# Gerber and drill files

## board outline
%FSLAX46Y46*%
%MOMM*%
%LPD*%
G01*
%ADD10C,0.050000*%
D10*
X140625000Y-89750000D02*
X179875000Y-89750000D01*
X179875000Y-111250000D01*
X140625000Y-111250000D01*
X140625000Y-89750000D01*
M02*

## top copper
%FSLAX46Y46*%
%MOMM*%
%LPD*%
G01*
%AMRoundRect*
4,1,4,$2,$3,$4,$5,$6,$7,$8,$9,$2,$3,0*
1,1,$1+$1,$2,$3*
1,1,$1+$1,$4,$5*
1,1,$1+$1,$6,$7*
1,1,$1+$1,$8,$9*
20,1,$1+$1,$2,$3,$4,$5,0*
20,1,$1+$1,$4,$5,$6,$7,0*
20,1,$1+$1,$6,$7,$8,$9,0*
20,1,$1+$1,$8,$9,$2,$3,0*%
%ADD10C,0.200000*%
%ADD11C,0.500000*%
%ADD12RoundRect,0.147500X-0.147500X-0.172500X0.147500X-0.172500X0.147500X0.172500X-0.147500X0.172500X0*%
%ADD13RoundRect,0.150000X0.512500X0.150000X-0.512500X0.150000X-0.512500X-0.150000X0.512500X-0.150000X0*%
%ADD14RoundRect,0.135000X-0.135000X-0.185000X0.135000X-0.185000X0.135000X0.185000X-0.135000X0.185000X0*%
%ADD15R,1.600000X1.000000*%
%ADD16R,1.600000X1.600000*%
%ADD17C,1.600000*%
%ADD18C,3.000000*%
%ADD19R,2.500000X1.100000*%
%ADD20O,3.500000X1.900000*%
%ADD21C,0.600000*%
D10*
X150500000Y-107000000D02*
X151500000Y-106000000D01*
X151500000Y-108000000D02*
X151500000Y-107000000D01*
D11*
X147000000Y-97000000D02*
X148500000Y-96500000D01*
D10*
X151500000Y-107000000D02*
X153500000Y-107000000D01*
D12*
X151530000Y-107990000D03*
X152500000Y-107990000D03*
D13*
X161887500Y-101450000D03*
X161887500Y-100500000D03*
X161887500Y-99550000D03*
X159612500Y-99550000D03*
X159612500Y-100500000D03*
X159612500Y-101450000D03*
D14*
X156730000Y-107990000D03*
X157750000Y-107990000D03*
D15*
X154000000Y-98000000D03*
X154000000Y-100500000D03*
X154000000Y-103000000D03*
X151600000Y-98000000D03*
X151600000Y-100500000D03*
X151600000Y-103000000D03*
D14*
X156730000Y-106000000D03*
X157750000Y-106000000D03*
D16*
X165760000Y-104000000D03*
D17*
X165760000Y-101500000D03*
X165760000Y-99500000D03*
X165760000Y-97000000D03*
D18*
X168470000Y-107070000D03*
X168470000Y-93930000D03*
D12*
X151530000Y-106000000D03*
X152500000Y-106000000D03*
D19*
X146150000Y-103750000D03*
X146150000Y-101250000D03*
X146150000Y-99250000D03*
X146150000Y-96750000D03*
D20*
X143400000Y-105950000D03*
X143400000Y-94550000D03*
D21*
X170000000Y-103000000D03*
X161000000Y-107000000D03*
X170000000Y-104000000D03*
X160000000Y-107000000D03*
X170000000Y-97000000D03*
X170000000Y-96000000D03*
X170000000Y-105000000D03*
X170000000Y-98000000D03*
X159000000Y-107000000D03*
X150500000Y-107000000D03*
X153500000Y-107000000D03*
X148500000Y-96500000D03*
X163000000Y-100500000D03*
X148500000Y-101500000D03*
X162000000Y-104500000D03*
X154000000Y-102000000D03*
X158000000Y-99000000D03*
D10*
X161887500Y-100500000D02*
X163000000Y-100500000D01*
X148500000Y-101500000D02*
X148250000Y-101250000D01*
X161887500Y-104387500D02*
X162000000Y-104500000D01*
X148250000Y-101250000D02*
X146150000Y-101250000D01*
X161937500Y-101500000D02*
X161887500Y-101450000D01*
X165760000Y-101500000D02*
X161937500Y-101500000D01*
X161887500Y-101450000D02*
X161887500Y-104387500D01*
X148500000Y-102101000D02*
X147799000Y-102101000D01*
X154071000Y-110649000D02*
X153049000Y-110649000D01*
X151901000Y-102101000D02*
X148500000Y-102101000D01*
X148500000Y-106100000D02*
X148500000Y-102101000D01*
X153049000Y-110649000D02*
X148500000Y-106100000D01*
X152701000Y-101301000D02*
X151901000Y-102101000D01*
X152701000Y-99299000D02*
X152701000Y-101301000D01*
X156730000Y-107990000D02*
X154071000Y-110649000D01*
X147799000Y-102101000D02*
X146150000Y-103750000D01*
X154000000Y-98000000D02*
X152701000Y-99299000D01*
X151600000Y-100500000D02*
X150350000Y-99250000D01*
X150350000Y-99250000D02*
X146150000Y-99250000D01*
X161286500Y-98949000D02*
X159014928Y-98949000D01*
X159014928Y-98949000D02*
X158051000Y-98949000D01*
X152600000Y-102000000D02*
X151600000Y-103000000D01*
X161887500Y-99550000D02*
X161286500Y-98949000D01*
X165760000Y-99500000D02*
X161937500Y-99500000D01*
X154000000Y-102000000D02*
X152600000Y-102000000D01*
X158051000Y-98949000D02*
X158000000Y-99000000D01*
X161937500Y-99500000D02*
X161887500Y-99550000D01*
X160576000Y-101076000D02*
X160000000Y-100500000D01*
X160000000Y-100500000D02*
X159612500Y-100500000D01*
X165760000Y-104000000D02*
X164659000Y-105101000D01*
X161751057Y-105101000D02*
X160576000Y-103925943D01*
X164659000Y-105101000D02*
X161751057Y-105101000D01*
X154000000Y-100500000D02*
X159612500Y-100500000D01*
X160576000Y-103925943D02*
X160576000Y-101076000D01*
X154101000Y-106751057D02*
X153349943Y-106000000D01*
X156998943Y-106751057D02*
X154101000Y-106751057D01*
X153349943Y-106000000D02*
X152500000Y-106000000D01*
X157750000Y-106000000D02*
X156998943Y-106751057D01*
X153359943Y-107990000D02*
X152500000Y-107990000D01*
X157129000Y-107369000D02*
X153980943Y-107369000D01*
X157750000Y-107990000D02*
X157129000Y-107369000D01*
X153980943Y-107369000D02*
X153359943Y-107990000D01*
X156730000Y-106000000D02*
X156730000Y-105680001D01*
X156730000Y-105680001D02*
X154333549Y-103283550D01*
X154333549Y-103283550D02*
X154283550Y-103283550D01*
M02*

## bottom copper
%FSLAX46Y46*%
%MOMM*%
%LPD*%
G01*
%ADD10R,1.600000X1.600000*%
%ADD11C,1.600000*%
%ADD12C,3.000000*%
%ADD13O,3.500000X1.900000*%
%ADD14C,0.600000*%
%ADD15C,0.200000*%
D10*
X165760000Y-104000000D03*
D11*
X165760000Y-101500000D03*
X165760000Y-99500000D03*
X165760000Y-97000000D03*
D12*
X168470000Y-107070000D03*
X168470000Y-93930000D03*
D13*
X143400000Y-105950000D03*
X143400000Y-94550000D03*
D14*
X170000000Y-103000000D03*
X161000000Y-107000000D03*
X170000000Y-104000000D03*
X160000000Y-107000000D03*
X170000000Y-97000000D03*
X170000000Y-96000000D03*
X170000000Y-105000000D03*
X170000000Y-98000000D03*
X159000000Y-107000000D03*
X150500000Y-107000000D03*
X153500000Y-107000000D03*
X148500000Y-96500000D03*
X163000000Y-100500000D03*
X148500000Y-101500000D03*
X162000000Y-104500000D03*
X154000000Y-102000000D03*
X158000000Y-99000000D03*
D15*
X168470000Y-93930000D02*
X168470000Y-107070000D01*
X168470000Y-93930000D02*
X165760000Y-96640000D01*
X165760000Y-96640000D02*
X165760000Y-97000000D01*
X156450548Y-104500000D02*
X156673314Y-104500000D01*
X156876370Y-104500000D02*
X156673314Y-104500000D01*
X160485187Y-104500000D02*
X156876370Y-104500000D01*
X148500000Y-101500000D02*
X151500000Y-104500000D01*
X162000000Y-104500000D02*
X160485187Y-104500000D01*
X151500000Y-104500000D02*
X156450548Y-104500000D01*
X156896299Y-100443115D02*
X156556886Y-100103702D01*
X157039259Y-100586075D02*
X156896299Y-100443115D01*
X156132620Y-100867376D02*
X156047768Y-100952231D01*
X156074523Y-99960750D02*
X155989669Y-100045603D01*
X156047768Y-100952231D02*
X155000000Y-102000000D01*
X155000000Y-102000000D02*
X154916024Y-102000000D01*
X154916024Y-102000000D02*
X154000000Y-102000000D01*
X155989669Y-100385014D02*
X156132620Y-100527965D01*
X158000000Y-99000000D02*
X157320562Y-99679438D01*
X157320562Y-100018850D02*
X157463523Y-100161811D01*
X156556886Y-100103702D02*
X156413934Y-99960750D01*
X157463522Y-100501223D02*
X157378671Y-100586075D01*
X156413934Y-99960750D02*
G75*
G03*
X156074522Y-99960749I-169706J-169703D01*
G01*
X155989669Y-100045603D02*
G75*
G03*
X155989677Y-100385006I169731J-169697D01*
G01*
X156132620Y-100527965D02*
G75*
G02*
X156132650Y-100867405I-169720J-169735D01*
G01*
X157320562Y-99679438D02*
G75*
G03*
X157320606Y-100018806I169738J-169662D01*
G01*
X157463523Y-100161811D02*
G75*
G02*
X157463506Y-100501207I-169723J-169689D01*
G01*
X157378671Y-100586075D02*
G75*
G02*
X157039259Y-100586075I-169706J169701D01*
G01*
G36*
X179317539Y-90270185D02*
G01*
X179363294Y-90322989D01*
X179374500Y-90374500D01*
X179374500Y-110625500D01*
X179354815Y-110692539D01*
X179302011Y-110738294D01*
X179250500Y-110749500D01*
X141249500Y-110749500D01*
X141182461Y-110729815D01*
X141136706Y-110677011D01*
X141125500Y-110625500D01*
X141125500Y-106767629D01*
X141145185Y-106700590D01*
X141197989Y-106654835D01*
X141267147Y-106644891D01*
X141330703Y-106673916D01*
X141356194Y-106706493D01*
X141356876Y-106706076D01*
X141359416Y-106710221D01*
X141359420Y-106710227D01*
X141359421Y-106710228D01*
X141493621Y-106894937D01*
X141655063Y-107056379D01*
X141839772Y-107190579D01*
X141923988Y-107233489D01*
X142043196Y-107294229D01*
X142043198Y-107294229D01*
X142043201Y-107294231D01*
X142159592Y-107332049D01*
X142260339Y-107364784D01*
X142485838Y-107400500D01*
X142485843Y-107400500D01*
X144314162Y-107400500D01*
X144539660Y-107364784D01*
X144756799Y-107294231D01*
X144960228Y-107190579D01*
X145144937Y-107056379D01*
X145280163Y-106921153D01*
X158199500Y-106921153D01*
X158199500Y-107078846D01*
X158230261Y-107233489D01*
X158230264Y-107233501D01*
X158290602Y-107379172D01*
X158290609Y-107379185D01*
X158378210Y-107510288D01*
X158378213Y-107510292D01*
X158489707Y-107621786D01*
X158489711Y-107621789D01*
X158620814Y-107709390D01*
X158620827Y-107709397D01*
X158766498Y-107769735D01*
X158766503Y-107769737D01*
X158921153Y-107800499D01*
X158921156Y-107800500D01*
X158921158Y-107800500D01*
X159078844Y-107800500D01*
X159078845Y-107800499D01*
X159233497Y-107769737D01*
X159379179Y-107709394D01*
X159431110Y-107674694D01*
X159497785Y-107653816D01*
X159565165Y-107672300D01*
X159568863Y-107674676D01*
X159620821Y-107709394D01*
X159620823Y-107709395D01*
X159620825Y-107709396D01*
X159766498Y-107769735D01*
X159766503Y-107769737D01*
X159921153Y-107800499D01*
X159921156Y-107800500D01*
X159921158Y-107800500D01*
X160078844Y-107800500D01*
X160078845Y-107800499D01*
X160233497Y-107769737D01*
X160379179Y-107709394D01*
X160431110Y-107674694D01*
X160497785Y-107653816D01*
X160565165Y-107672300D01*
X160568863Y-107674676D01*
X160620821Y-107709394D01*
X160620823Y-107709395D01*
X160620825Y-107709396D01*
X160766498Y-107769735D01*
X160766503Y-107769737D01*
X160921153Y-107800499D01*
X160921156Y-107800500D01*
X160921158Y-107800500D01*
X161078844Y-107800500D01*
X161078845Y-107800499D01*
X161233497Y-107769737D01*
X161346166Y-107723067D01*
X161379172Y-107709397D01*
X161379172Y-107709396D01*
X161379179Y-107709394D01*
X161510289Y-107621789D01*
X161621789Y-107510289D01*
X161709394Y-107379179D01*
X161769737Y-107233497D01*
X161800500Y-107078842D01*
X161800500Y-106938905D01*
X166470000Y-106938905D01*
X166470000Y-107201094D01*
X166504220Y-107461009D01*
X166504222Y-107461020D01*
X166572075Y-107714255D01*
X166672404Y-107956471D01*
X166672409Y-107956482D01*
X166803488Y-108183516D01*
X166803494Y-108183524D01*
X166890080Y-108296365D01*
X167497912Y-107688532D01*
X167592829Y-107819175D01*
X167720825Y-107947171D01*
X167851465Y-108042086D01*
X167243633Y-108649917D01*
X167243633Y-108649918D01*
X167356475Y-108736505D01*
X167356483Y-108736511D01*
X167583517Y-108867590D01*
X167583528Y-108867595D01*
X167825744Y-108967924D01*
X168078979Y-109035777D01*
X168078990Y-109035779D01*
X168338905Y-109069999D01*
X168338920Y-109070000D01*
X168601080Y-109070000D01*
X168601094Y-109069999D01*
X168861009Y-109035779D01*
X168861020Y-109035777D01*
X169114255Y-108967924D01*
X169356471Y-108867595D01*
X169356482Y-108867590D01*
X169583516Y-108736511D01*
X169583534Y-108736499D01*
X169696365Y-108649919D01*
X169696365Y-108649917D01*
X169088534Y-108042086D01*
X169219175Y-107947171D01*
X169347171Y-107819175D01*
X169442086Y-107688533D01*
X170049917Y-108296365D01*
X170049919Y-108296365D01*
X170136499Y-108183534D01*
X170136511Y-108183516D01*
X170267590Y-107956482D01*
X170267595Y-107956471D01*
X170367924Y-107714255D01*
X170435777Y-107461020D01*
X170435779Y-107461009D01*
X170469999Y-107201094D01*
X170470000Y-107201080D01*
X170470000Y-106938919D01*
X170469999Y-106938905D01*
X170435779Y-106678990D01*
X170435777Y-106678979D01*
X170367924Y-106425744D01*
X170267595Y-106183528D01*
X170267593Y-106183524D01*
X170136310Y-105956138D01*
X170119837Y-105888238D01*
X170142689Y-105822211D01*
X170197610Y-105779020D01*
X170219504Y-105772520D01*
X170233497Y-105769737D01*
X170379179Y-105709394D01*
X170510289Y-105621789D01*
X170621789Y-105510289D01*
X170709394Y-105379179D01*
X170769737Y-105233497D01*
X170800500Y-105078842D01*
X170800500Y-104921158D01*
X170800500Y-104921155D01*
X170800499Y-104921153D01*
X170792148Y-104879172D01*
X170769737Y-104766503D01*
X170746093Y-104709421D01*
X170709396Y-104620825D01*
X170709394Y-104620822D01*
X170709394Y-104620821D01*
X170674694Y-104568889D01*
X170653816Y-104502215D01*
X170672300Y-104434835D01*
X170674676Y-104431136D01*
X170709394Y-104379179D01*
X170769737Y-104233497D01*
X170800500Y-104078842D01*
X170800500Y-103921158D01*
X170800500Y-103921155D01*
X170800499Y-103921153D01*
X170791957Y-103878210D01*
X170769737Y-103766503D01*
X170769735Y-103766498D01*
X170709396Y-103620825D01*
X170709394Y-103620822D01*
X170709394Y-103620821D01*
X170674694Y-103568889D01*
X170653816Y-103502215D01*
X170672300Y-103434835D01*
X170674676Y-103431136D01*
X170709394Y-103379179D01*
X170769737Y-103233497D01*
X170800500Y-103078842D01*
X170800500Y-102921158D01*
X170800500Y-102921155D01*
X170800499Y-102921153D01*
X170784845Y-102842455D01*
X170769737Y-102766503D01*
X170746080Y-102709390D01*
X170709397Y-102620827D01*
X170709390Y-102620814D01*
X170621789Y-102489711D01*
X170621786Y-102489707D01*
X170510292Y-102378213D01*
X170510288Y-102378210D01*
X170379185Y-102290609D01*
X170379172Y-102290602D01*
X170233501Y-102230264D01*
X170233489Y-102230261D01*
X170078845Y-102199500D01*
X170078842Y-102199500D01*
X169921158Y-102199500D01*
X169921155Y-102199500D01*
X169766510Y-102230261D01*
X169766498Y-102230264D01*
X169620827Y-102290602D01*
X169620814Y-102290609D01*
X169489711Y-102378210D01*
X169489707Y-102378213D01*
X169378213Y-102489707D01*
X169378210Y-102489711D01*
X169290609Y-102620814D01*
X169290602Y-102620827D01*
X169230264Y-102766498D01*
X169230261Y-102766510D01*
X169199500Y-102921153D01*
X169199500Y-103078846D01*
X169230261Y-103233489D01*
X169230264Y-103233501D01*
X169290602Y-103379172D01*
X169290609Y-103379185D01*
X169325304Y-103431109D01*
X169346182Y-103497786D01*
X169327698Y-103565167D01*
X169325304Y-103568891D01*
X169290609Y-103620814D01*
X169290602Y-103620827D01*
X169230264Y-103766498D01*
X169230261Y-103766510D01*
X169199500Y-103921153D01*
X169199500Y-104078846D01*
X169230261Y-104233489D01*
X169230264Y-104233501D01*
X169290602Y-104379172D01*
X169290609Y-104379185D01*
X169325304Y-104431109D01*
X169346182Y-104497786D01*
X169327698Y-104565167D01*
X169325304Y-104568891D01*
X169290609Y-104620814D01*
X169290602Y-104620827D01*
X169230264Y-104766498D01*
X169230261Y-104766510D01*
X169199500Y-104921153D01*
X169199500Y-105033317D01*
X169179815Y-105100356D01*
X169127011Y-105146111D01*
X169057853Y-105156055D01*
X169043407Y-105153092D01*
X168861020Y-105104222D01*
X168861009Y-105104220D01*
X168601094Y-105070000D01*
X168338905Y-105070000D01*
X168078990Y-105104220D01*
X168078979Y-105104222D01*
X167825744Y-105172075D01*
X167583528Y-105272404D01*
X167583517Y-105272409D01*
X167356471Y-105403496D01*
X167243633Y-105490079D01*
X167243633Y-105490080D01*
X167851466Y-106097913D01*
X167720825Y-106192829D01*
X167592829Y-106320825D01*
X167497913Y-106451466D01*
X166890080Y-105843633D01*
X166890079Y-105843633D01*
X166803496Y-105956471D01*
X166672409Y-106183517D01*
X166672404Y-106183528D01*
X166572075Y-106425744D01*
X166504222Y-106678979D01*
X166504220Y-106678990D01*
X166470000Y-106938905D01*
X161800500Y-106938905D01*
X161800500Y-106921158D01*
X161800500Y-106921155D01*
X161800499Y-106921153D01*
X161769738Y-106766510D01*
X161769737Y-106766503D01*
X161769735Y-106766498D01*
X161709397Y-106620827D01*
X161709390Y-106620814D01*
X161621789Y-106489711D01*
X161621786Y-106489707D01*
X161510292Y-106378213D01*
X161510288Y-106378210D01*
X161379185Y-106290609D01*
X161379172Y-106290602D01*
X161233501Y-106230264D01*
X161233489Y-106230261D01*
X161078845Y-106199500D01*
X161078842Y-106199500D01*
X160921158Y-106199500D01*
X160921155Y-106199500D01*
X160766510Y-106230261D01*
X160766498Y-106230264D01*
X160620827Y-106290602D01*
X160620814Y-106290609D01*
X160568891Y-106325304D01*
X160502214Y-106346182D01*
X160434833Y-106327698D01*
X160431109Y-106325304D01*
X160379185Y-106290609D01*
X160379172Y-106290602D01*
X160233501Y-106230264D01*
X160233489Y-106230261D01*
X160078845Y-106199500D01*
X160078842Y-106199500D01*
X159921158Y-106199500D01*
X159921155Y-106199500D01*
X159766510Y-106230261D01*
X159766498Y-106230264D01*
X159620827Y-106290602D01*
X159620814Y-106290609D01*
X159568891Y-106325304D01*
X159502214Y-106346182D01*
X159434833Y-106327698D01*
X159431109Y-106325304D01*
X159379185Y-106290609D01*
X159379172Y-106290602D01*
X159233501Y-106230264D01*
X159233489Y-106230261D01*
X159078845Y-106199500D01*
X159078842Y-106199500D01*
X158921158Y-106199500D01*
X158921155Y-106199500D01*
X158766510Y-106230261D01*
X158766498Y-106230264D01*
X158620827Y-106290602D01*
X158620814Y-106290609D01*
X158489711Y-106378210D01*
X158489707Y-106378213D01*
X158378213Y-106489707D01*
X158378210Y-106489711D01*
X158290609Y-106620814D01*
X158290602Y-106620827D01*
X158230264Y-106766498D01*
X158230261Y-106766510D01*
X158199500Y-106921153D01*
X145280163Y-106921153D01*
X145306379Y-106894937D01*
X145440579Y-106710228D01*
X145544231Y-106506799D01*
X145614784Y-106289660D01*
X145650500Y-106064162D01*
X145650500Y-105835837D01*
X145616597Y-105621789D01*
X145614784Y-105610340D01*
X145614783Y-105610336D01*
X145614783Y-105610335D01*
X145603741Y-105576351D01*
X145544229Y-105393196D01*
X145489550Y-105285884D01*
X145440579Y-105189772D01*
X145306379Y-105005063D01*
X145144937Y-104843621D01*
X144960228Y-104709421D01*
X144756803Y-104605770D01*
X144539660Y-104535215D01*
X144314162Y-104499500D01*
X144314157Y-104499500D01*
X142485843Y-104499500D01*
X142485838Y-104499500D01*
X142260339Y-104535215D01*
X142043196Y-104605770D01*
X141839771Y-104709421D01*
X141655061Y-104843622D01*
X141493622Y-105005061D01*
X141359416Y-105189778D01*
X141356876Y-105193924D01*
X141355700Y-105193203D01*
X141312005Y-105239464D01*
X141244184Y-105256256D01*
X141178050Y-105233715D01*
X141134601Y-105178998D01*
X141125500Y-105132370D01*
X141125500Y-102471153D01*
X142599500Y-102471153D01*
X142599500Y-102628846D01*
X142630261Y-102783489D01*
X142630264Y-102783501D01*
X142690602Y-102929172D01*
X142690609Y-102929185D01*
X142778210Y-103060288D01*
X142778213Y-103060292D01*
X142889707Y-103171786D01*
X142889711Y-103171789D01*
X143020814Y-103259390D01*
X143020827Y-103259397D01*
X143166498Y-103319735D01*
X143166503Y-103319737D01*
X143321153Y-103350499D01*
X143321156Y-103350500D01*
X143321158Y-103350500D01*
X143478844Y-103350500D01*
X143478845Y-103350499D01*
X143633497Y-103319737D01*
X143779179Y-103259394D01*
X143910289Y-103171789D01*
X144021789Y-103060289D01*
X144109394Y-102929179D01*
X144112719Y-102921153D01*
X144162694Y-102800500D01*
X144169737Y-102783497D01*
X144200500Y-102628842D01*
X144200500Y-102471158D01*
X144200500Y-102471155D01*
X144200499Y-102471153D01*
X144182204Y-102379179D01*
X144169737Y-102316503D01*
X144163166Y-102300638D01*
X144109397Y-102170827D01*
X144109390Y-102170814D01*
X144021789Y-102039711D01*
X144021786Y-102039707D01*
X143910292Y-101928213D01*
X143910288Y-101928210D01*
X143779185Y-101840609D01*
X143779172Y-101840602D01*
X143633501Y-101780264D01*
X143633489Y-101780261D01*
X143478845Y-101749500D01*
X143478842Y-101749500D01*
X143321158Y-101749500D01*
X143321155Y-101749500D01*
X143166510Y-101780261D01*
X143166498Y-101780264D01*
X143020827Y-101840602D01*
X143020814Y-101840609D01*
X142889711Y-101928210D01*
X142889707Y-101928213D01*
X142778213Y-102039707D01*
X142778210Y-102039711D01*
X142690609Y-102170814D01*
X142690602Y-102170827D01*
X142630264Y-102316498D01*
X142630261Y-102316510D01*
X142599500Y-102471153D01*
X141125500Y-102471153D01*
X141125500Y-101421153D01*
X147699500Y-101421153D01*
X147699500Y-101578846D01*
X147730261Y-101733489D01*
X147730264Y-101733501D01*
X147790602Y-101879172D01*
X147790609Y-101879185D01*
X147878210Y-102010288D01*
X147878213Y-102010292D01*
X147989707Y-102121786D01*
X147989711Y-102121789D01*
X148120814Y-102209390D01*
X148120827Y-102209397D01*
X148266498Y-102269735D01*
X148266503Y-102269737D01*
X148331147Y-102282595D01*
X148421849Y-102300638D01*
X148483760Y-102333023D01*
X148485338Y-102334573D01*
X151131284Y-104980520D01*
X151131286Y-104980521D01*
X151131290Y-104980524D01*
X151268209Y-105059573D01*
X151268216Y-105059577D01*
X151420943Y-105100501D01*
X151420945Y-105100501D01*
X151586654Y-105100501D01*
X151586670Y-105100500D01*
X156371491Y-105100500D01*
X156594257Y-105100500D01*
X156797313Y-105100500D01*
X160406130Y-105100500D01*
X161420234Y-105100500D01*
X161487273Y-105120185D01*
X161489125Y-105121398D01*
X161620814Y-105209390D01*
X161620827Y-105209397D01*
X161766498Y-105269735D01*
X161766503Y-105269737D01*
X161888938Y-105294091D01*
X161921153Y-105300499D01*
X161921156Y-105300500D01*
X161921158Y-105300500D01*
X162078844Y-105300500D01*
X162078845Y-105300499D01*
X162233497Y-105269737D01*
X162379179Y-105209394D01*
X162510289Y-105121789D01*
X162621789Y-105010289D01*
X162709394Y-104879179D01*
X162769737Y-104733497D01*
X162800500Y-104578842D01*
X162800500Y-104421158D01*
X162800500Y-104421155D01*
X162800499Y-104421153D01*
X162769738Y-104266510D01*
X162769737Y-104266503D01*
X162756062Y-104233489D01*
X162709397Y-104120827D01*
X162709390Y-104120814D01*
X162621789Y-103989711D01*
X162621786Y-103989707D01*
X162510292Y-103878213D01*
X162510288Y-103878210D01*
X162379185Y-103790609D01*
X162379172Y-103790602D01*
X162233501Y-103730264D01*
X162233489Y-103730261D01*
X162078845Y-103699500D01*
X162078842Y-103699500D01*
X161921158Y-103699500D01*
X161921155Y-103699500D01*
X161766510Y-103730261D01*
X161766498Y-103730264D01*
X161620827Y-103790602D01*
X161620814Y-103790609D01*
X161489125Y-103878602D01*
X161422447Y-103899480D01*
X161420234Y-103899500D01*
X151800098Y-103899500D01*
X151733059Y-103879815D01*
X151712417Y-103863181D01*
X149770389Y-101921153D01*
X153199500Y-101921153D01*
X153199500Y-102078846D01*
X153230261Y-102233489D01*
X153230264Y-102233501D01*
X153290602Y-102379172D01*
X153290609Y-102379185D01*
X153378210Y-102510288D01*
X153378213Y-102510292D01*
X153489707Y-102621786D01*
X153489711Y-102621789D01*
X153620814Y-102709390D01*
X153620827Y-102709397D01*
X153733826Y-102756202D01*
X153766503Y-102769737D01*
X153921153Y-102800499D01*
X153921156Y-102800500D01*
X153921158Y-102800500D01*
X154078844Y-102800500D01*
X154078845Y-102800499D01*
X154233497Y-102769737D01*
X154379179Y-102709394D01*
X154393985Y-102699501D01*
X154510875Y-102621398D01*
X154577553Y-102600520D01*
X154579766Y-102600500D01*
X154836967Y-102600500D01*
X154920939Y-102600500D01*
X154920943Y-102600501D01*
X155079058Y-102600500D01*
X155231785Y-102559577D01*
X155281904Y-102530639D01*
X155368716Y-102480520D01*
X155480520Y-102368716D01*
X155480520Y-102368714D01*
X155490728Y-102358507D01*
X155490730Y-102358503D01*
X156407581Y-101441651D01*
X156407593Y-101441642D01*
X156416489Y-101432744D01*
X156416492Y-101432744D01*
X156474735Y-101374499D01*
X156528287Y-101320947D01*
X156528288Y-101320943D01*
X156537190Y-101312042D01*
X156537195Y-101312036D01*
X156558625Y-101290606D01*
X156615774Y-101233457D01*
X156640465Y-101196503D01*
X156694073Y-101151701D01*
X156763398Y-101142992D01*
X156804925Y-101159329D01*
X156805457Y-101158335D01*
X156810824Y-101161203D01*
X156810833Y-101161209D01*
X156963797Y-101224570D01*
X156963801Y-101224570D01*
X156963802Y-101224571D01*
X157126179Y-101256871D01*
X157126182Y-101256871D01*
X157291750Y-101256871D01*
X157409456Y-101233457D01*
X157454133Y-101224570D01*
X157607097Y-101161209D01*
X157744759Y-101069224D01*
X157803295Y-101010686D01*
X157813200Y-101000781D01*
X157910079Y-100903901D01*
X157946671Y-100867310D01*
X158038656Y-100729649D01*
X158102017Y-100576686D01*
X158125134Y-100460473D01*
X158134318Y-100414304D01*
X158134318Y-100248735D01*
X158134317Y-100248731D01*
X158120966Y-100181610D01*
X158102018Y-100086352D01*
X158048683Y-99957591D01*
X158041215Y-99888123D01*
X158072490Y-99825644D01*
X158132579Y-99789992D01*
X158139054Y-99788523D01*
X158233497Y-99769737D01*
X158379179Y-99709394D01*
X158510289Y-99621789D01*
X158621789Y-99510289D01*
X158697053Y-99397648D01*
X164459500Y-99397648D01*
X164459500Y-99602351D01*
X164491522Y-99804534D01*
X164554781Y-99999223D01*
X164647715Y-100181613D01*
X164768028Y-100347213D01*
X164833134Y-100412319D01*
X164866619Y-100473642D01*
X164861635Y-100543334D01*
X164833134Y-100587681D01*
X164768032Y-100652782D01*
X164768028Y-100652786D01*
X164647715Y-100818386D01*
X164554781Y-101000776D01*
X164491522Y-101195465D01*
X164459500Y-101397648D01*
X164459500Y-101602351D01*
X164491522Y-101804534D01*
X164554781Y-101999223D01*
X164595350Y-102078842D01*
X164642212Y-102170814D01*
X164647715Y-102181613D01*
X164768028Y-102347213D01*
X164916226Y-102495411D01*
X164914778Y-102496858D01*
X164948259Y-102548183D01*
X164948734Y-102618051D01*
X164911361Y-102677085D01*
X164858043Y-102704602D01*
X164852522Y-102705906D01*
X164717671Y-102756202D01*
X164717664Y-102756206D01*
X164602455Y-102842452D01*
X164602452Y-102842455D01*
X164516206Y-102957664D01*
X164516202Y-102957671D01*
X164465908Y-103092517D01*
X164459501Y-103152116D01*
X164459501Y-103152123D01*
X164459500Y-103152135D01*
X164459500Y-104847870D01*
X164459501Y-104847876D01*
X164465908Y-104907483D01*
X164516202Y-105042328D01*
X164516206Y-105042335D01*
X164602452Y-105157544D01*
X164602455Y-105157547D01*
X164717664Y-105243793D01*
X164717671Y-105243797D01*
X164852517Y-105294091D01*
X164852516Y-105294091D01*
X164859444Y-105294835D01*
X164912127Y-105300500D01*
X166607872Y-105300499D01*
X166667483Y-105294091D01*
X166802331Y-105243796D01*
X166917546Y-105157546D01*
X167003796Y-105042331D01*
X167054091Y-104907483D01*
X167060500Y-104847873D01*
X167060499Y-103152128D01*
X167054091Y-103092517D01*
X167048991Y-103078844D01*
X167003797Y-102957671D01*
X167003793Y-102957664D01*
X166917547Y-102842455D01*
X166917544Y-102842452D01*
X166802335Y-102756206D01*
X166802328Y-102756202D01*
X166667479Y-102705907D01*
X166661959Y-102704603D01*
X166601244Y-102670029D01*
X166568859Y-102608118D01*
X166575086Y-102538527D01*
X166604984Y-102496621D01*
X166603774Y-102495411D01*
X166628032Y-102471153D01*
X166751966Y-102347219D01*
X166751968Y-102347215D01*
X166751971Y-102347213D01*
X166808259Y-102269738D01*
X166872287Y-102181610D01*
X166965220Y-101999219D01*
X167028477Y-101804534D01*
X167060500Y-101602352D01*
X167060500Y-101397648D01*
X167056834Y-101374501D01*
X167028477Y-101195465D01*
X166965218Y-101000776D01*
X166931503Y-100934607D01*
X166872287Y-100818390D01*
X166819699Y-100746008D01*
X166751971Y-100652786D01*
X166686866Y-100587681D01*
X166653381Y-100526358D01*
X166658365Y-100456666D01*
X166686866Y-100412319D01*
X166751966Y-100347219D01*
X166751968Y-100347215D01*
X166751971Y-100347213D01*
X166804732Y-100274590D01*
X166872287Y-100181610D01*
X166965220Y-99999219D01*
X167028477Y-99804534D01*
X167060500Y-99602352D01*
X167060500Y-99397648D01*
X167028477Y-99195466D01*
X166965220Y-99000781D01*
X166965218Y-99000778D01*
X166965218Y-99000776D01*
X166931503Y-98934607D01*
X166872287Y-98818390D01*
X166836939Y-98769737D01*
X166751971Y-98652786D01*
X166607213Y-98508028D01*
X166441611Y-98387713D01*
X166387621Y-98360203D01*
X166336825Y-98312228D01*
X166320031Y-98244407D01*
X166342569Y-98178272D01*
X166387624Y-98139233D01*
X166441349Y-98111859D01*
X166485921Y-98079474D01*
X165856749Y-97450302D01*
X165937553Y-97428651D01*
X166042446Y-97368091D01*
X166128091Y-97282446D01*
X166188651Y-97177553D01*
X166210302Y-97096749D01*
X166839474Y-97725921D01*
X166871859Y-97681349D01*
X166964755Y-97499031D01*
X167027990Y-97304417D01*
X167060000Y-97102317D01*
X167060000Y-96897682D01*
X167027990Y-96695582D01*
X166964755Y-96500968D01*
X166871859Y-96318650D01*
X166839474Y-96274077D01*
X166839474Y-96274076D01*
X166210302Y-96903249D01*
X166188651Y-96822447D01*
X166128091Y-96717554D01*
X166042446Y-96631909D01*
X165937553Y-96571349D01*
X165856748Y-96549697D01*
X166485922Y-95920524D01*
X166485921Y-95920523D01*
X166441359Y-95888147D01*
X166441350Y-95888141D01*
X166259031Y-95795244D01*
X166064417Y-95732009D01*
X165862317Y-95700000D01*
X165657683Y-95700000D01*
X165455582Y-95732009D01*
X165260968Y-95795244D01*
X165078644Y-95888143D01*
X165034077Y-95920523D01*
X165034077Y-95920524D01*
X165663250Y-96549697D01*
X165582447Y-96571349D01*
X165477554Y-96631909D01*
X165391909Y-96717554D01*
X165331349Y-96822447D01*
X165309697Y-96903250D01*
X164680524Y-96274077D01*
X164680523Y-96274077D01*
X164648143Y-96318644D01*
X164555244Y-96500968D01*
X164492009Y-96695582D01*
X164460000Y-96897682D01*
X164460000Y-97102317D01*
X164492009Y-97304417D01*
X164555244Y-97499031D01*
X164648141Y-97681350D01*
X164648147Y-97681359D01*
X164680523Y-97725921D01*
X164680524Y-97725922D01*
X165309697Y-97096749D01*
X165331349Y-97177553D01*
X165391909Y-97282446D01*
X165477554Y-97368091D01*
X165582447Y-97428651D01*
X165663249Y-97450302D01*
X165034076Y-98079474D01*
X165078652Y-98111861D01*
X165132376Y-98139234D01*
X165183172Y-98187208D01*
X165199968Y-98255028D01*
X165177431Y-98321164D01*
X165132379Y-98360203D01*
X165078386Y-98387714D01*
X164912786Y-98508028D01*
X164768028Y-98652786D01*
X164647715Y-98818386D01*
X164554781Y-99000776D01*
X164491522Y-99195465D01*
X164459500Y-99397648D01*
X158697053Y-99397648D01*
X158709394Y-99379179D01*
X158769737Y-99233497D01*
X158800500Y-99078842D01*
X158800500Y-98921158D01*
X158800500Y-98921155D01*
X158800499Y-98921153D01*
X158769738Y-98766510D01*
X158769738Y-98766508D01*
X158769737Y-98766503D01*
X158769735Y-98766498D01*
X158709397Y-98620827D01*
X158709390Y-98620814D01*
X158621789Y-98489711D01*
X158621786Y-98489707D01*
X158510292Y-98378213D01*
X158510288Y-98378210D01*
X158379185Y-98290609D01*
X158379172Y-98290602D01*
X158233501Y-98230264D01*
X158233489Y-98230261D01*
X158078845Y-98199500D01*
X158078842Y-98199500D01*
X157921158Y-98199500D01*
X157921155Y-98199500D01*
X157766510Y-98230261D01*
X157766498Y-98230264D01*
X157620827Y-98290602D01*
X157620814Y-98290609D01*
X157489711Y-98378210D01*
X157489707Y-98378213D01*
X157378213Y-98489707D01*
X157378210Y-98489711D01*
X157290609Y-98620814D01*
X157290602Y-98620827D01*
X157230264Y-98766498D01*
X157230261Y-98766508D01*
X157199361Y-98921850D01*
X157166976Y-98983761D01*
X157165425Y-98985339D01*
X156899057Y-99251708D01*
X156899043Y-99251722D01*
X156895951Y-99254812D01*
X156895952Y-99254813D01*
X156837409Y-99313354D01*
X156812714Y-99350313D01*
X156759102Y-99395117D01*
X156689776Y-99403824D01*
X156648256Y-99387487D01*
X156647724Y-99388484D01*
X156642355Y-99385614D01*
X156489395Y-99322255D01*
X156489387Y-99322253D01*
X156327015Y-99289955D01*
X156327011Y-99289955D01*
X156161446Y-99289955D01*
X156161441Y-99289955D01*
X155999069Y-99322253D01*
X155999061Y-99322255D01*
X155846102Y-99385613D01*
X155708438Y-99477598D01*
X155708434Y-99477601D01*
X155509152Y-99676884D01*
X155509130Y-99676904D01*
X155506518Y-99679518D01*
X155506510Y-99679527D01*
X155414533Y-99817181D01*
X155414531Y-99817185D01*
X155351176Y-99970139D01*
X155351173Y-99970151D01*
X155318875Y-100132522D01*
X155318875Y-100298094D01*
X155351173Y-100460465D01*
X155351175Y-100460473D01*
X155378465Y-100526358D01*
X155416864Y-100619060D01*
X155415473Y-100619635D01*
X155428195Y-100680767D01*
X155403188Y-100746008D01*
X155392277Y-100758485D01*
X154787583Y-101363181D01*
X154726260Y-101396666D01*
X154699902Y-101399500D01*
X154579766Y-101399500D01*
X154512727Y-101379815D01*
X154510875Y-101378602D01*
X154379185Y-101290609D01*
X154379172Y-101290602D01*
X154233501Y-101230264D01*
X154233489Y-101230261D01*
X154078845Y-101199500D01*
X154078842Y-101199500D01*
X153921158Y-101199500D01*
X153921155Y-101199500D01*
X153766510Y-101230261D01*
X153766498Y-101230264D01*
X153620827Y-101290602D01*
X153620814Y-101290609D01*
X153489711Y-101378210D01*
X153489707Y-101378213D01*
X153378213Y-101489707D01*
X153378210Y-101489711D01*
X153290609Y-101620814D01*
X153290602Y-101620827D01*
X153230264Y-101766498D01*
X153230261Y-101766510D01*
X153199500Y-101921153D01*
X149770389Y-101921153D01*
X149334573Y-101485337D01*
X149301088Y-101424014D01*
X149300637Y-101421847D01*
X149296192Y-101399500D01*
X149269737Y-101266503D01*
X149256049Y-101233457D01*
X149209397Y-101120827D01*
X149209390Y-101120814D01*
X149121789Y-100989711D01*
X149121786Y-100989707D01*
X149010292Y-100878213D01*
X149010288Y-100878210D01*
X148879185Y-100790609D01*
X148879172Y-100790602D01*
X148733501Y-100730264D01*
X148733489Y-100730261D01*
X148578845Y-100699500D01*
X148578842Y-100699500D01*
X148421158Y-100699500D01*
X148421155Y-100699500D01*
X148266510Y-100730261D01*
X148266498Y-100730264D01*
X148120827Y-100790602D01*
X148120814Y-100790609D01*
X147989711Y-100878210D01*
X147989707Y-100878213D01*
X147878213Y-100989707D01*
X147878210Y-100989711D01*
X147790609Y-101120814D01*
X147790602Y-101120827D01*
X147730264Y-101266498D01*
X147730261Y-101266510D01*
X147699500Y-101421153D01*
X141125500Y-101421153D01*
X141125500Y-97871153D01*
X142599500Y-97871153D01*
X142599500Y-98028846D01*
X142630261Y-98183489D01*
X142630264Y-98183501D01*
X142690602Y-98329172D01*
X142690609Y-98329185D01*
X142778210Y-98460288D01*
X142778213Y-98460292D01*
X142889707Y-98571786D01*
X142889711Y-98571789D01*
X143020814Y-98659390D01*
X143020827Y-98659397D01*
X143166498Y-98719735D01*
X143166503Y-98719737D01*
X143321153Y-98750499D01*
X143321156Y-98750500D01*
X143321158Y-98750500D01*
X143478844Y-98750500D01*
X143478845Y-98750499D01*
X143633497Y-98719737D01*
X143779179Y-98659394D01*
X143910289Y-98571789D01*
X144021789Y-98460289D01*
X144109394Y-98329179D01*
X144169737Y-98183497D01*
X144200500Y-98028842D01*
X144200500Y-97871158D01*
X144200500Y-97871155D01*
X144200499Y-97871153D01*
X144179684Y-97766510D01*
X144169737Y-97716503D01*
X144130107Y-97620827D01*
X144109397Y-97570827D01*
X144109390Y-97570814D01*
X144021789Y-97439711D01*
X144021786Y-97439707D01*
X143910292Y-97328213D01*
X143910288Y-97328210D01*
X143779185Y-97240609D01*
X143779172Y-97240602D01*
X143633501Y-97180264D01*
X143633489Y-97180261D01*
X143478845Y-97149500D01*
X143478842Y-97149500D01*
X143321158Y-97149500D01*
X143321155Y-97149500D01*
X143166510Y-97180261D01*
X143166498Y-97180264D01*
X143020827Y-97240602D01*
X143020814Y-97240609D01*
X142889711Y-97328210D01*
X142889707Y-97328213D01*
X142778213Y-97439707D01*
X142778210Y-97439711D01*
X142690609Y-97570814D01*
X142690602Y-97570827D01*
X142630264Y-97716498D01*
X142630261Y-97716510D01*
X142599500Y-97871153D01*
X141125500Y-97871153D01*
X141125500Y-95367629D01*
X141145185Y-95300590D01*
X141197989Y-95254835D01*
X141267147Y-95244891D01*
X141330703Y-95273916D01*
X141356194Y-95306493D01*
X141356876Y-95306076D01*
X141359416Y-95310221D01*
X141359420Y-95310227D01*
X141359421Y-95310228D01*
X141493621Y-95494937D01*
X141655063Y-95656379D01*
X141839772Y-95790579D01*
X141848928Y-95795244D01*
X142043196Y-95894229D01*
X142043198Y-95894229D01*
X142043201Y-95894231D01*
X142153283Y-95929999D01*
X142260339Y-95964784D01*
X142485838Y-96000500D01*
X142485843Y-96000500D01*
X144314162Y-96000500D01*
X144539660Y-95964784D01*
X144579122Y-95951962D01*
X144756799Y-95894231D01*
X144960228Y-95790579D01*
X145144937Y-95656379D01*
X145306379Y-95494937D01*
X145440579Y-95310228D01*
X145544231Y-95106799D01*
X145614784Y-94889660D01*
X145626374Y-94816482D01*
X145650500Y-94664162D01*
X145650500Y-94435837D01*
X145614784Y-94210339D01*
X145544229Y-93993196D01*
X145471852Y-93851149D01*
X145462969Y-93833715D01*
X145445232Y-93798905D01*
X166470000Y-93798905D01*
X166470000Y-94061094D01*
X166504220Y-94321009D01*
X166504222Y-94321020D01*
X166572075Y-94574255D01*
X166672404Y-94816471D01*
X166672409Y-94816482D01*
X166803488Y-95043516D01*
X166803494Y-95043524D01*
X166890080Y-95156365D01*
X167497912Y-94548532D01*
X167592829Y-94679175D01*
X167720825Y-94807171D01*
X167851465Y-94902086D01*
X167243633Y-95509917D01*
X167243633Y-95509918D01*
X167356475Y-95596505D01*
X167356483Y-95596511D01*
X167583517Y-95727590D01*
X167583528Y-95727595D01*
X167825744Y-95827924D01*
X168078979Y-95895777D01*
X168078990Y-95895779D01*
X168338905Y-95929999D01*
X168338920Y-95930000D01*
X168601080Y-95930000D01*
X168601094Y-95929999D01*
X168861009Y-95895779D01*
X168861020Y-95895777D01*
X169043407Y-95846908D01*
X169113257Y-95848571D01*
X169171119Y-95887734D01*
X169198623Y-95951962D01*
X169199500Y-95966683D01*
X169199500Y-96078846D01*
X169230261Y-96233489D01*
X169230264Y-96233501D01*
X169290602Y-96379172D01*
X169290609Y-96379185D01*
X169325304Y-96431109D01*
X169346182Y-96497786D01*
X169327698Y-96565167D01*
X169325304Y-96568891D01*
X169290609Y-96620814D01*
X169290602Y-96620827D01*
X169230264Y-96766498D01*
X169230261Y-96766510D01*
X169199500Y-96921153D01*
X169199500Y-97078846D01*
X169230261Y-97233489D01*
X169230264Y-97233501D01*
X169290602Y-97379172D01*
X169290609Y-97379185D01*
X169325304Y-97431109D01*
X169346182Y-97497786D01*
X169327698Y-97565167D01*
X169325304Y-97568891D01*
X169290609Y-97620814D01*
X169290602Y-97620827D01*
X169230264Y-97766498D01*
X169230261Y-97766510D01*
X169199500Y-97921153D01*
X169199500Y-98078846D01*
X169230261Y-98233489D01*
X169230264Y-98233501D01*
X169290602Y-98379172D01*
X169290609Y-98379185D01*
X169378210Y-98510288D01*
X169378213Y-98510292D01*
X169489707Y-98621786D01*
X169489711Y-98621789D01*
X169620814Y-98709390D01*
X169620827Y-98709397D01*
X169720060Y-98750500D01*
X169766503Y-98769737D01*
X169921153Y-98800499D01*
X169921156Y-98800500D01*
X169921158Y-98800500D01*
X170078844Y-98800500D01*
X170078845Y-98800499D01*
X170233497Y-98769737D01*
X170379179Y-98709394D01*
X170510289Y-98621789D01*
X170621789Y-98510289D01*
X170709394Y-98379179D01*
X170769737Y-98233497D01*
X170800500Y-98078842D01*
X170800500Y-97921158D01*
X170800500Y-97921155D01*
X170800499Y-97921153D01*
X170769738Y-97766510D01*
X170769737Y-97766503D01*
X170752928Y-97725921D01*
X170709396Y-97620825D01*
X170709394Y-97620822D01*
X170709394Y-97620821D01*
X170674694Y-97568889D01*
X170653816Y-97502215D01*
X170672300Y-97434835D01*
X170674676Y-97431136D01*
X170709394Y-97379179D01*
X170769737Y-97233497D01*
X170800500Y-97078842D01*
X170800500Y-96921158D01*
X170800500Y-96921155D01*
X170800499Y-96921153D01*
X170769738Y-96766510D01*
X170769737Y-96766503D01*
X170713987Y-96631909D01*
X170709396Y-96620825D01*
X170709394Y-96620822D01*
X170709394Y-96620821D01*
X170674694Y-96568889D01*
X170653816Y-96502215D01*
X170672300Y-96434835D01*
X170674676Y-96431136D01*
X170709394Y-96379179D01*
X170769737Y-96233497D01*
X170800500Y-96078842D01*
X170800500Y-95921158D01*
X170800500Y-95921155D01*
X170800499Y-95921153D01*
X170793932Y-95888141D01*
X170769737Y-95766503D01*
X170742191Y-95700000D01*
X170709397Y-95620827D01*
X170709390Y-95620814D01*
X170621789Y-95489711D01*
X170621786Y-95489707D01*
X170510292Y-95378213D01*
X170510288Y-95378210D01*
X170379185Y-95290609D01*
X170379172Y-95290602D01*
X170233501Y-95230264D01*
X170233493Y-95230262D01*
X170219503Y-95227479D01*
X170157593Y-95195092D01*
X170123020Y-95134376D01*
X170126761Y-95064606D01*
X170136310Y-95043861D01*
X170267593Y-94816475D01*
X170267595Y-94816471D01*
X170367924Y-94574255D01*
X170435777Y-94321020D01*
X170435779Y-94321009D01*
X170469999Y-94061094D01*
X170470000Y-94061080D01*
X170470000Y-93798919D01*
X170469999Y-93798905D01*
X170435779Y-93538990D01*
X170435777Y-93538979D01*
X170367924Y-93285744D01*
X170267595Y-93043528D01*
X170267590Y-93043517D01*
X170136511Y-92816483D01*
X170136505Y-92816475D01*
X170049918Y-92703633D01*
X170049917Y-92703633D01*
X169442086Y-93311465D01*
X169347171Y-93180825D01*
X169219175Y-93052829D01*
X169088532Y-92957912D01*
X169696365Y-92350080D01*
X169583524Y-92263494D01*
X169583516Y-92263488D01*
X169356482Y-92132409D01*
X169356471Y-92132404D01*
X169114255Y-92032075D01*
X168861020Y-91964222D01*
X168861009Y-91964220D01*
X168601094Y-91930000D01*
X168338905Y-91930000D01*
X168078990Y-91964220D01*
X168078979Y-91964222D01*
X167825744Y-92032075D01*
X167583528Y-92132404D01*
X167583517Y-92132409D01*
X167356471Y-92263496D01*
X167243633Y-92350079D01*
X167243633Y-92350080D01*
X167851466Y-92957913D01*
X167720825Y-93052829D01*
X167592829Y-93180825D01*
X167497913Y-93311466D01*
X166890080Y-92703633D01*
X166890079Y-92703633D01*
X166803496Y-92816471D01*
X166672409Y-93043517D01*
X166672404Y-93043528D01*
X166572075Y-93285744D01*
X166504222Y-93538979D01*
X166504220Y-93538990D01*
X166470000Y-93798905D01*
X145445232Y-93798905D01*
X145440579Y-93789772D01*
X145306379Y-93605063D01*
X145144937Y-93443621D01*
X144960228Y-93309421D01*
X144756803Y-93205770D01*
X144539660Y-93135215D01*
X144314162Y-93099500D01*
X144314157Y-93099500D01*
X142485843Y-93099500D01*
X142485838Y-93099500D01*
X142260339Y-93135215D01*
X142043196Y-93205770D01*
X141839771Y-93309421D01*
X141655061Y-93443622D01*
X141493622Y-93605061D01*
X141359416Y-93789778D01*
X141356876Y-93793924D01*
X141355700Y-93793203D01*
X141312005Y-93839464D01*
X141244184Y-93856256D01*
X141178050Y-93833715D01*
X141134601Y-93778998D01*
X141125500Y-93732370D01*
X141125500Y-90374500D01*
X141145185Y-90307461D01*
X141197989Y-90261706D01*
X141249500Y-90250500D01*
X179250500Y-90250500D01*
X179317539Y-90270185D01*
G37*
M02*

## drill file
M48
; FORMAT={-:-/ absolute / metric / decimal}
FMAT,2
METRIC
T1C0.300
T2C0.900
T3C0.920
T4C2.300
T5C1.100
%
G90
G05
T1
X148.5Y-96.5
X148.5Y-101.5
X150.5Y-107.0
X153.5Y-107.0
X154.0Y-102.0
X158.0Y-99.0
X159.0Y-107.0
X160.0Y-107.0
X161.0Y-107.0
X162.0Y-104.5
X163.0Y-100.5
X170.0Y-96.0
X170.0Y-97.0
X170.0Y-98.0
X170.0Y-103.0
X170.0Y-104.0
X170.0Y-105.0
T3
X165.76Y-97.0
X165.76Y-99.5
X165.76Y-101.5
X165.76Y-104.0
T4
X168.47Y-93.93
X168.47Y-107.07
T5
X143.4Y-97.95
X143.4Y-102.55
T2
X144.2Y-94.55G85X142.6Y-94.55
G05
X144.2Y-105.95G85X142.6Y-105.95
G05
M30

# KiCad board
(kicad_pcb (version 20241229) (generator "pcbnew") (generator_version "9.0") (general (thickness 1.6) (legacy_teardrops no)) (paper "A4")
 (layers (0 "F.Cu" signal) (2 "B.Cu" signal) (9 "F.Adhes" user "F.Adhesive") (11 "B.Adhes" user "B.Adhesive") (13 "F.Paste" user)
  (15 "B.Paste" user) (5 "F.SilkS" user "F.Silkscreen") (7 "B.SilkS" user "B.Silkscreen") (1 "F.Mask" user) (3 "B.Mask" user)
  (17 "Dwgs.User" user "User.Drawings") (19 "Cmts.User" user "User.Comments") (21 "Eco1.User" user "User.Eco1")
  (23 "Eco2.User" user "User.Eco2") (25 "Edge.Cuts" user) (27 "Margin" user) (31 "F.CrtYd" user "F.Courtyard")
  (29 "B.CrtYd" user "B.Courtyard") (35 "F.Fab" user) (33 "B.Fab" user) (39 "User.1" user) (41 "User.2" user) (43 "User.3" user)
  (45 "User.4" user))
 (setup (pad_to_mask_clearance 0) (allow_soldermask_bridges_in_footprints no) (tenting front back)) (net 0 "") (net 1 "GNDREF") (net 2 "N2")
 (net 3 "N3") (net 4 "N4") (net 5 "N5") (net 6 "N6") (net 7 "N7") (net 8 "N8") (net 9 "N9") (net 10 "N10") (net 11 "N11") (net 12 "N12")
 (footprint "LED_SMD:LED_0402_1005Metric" (layer "F.Cu") (at 152.015 107.99)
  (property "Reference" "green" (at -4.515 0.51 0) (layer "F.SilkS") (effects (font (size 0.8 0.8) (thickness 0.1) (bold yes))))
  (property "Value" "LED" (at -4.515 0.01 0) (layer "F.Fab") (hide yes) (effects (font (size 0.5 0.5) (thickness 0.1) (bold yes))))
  (pad "1" smd roundrect (at -0.485 0) (size 0.59 0.64) (layers "F.Cu" "F.Mask" "F.Paste") (roundrect_rratio 0.25) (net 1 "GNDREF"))
  (pad "2" smd roundrect (at 0.485 0) (size 0.59 0.64) (layers "F.Cu" "F.Mask" "F.Paste") (roundrect_rratio 0.25) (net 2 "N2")))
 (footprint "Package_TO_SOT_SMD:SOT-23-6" (layer "F.Cu") (at 160.75 100.5 180)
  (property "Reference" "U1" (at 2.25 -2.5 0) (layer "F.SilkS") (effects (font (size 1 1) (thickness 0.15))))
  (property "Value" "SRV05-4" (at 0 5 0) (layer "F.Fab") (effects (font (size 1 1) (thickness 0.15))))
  (pad "1" smd roundrect (at -1.1375 -0.95 180) (size 1.325 0.6) (layers "F.Cu" "F.Mask" "F.Paste") (roundrect_rratio 0.25) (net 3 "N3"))
  (pad "2" smd roundrect (at -1.1375 0 180) (size 1.325 0.6) (layers "F.Cu" "F.Mask" "F.Paste") (roundrect_rratio 0.25) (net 1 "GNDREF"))
  (pad "3" smd roundrect (at -1.1375 0.95 180) (size 1.325 0.6) (layers "F.Cu" "F.Mask" "F.Paste") (roundrect_rratio 0.25) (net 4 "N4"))
  (pad "4" smd roundrect (at 1.1375 0.95 180) (size 1.325 0.6) (layers "F.Cu" "F.Mask" "F.Paste") (roundrect_rratio 0.25) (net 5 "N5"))
  (pad "5" smd roundrect (at 1.1375 0 180) (size 1.325 0.6) (layers "F.Cu" "F.Mask" "F.Paste") (roundrect_rratio 0.25) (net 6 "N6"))
  (pad "6" smd roundrect (at 1.1375 -0.95 180) (size 1.325 0.6) (layers "F.Cu" "F.Mask" "F.Paste") (roundrect_rratio 0.25) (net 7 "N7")))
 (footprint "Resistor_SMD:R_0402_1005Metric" (layer "F.Cu") (at 157.24 107.99)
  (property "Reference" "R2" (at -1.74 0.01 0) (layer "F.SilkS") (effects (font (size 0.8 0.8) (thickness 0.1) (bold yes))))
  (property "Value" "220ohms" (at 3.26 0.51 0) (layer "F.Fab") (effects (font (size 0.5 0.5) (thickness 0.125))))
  (pad "1" smd roundrect (at -0.51 0) (size 0.54 0.64) (layers "F.Cu" "F.Mask" "F.Paste") (roundrect_rratio 0.25) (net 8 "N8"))
  (pad "2" smd roundrect (at 0.51 0) (size 0.54 0.64) (layers "F.Cu" "F.Mask" "F.Paste") (roundrect_rratio 0.25) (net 2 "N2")))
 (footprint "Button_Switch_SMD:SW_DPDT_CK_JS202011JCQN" (layer "F.Cu") (at 152.8 100.5 -90)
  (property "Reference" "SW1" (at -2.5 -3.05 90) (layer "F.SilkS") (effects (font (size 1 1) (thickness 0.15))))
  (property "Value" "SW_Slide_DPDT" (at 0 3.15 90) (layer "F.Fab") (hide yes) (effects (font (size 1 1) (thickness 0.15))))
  (pad "1" smd rect (at -2.5 -1.2 270) (size 1 1.6) (layers "F.Cu" "F.Mask" "F.Paste") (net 8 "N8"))
  (pad "2" smd rect (at 0 -1.2 270) (size 1 1.6) (layers "F.Cu" "F.Mask" "F.Paste") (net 6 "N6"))
  (pad "3" smd rect (at 2.5 -1.2 270) (size 1 1.6) (layers "F.Cu" "F.Mask" "F.Paste") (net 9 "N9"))
  (pad "4" smd rect (at -2.5 1.2 270) (size 1 1.6) (layers "F.Cu" "F.Mask" "F.Paste") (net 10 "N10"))
  (pad "5" smd rect (at 0 1.2 270) (size 1 1.6) (layers "F.Cu" "F.Mask" "F.Paste") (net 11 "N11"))
  (pad "6" smd rect (at 2.5 1.2 270) (size 1 1.6) (layers "F.Cu" "F.Mask" "F.Paste") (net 4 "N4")))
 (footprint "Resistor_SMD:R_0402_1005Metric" (layer "F.Cu") (at 157.24 106)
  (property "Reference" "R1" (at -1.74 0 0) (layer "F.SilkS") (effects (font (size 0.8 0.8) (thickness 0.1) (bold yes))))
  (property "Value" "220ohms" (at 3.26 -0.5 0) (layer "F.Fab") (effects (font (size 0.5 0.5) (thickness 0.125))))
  (pad "1" smd roundrect (at -0.51 0) (size 0.54 0.64) (layers "F.Cu" "F.Mask" "F.Paste") (roundrect_rratio 0.25) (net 9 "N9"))
  (pad "2" smd roundrect (at 0.51 0) (size 0.54 0.64) (layers "F.Cu" "F.Mask" "F.Paste") (roundrect_rratio 0.25) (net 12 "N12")))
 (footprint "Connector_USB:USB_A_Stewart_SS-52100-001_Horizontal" (layer "F.Cu") (at 165.76 104 90)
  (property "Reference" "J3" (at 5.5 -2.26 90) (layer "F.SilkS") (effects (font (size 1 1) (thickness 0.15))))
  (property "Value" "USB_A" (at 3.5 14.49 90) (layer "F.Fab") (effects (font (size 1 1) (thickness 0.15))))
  (pad "1" thru_hole rect (at 0 0 90) (size 1.6 1.6) (drill 0.92) (layers "*.Cu" "*.Mask") (remove_unused_layers no) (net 6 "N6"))
  (pad "2" thru_hole circle (at 2.5 0 90) (size 1.6 1.6) (drill 0.92) (layers "*.Cu" "*.Mask") (remove_unused_layers no) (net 3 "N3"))
  (pad "3" thru_hole circle (at 4.5 0 90) (size 1.6 1.6) (drill 0.92) (layers "*.Cu" "*.Mask") (remove_unused_layers no) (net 4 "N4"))
  (pad "4" thru_hole circle (at 7 0 90) (size 1.6 1.6) (drill 0.92) (layers "*.Cu" "*.Mask") (remove_unused_layers no) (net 1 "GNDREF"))
  (pad "5" thru_hole circle (at -3.07 2.71 90) (size 3 3) (drill 2.3) (layers "*.Cu" "*.Mask") (remove_unused_layers no) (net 1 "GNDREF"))
  (pad "5" thru_hole circle (at 10.07 2.71 90) (size 3 3) (drill 2.3) (layers "*.Cu" "*.Mask") (remove_unused_layers no) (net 1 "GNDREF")))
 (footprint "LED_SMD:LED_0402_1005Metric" (layer "F.Cu") (at 152.015 106)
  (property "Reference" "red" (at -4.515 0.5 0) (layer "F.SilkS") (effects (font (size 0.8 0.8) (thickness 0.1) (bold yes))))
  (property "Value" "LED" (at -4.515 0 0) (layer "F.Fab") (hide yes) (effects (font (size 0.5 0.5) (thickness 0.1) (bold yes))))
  (pad "1" smd roundrect (at -0.485 0) (size 0.59 0.64) (layers "F.Cu" "F.Mask" "F.Paste") (roundrect_rratio 0.25) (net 1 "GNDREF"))
  (pad "2" smd roundrect (at 0.485 0) (size 0.59 0.64) (layers "F.Cu" "F.Mask" "F.Paste") (roundrect_rratio 0.25) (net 12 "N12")))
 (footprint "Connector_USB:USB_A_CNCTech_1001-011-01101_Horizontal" (layer "F.Cu") (at 136.5 100.25 180)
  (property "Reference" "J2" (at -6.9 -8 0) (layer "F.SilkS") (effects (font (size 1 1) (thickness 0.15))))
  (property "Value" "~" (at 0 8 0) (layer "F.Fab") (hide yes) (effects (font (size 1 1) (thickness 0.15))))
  (pad "" np_thru_hole circle (at -6.9 -2.3 180) (size 1.1 1.1) (drill 1.1) (layers "*.Cu" "*.Mask"))
  (pad "" np_thru_hole circle (at -6.9 2.3 180) (size 1.1 1.1) (drill 1.1) (layers "*.Cu" "*.Mask"))
  (pad "1" smd rect (at -9.65 -3.5 180) (size 2.5 1.1) (layers "F.Cu" "F.Mask" "F.Paste") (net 8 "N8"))
  (pad "2" smd rect (at -9.65 -1 180) (size 2.5 1.1) (layers "F.Cu" "F.Mask" "F.Paste") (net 3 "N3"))
  (pad "3" smd rect (at -9.65 1 180) (size 2.5 1.1) (layers "F.Cu" "F.Mask" "F.Paste") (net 11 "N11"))
  (pad "4" smd rect (at -9.65 3.5 180) (size 2.5 1.1) (layers "F.Cu" "F.Mask" "F.Paste") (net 1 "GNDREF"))
  (pad "5" thru_hole oval (at -6.9 -5.7 180) (size 3.5 1.9) (drill oval 2.5 0.9) (layers "*.Cu" "*.Mask") (remove_unused_layers no))
  (pad "5" thru_hole oval (at -6.9 5.7 180) (size 3.5 1.9) (drill oval 2.5 0.9) (layers "*.Cu" "*.Mask") (remove_unused_layers no)))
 (gr_line (start 150.5 107) (end 151.5 106) (stroke (width 0.2) (type default)) (layer "F.Cu") (net 1))
 (gr_line (start 151.5 108) (end 151.5 107) (stroke (width 0.2) (type default)) (layer "F.Cu") (net 1))
 (gr_line (start 147 97) (end 148.5 96.5) (stroke (width 0.5) (type solid)) (layer "F.Cu") (net 1))
 (gr_line (start 151.5 107) (end 153.5 107) (stroke (width 0.2) (type default)) (layer "F.Cu") (net 1))
 (gr_rect (start 140.625 89.75) (end 179.875 111.25) (stroke (width 0.05) (type default)) (fill no) (layer "Edge.Cuts"))
 (via (at 170 103) (size 0.6) (drill 0.3) (layers "F.Cu" "B.Cu") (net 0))
 (via (at 161 107) (size 0.6) (drill 0.3) (layers "F.Cu" "B.Cu") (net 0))
 (via (at 170 104) (size 0.6) (drill 0.3) (layers "F.Cu" "B.Cu") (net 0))
 (via (at 160 107) (size 0.6) (drill 0.3) (layers "F.Cu" "B.Cu") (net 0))
 (via (at 170 97) (size 0.6) (drill 0.3) (layers "F.Cu" "B.Cu") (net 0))
 (via (at 170 96) (size 0.6) (drill 0.3) (layers "F.Cu" "B.Cu") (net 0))
 (via (at 170 105) (size 0.6) (drill 0.3) (layers "F.Cu" "B.Cu") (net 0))
 (via (at 170 98) (size 0.6) (drill 0.3) (layers "F.Cu" "B.Cu") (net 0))
 (via (at 159 107) (size 0.6) (drill 0.3) (layers "F.Cu" "B.Cu") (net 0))
 (segment (start 161.8875 100.5) (end 163 100.5) (width 0.2) (layer "F.Cu") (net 1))
 (via (at 150.5 107) (size 0.6) (drill 0.3) (layers "F.Cu" "B.Cu") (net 1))
 (via (at 153.5 107) (size 0.6) (drill 0.3) (layers "F.Cu" "B.Cu") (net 1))
 (via (at 148.5 96.5) (size 0.6) (drill 0.3) (layers "F.Cu" "B.Cu") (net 1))
 (via (at 163 100.5) (size 0.6) (drill 0.3) (layers "F.Cu" "B.Cu") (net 1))
 (segment (start 168.47 93.93) (end 168.47 107.07) (width 0.2) (layer "B.Cu") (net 1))
 (segment (start 168.47 93.93) (end 165.76 96.64) (width 0.2) (layer "B.Cu") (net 1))
 (segment (start 165.76 96.64) (end 165.76 97) (width 0.2) (layer "B.Cu") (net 1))
 (segment (start 148.5 101.5) (end 148.25 101.25) (width 0.2) (layer "F.Cu") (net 3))
 (segment (start 161.8875 104.3875) (end 162 104.5) (width 0.2) (layer "F.Cu") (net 3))
 (segment (start 148.25 101.25) (end 146.15 101.25) (width 0.2) (layer "F.Cu") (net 3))
 (segment (start 161.9375 101.5) (end 161.8875 101.45) (width 0.2) (layer "F.Cu") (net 3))
 (segment (start 165.76 101.5) (end 161.9375 101.5) (width 0.2) (layer "F.Cu") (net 3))
 (segment (start 161.8875 101.45) (end 161.8875 104.3875) (width 0.2) (layer "F.Cu") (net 3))
 (via (at 148.5 101.5) (size 0.6) (drill 0.3) (layers "F.Cu" "B.Cu") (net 3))
 (via (at 162 104.5) (size 0.6) (drill 0.3) (layers "F.Cu" "B.Cu")
  (teardrops (best_length_ratio 0.6) (max_length 1) (best_width_ratio 1) (max_width 2) (curved_edges no) (filter_ratio 0.9) (enabled no)
   (allow_two_segments yes) (prefer_zone_connections yes))
  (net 3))
 (segment (start 156.450548 104.5) (end 156.673314 104.5) (width 0.2) (layer "B.Cu") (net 3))
 (segment (start 156.87637 104.5) (end 156.673314 104.5) (width 0.2) (layer "B.Cu") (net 3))
 (segment (start 160.485187 104.5) (end 156.87637 104.5) (width 0.2) (layer "B.Cu") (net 3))
 (segment (start 148.5 101.5) (end 151.5 104.5) (width 0.2) (layer "B.Cu") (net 3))
 (segment (start 162 104.5) (end 160.485187 104.5) (width 0.2) (layer "B.Cu") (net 3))
 (segment (start 151.5 104.5) (end 156.450548 104.5) (width 0.2) (layer "B.Cu") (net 3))
 (segment (start 148.5 102.101) (end 147.799 102.101) (width 0.2) (layer "F.Cu") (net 8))
 (segment (start 154.071 110.649) (end 153.049 110.649) (width 0.2) (layer "F.Cu") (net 8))
 (segment (start 151.901 102.101) (end 148.5 102.101) (width 0.2) (layer "F.Cu") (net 8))
 (segment (start 148.5 106.1) (end 148.5 102.101) (width 0.2) (layer "F.Cu") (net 8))
 (segment (start 153.049 110.649) (end 148.5 106.1) (width 0.2) (layer "F.Cu") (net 8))
 (segment (start 152.701 101.301) (end 151.901 102.101) (width 0.2) (layer "F.Cu") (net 8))
 (segment (start 152.701 99.299) (end 152.701 101.301) (width 0.2) (layer "F.Cu") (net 8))
 (segment (start 156.73 107.99) (end 154.071 110.649) (width 0.2) (layer "F.Cu") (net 8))
 (segment (start 147.799 102.101) (end 146.15 103.75) (width 0.2) (layer "F.Cu") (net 8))
 (segment (start 154 98) (end 152.701 99.299) (width 0.2) (layer "F.Cu") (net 8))
 (segment (start 151.6 100.5) (end 150.35 99.25) (width 0.2) (layer "F.Cu") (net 11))
 (segment (start 150.35 99.25) (end 146.15 99.25) (width 0.2) (layer "F.Cu") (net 11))
 (segment (start 161.2865 98.949) (end 159.014928 98.949) (width 0.2) (layer "F.Cu") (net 4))
 (segment (start 159.014928 98.949) (end 158.051 98.949) (width 0.2) (layer "F.Cu") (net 4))
 (segment (start 152.6 102) (end 151.6 103) (width 0.2) (layer "F.Cu") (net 4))
 (segment (start 161.8875 99.55) (end 161.2865 98.949) (width 0.2) (layer "F.Cu") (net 4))
 (segment (start 165.76 99.5) (end 161.9375 99.5) (width 0.2) (layer "F.Cu") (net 4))
 (segment (start 154 102) (end 152.6 102) (width 0.2) (layer "F.Cu") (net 4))
 (segment (start 158.051 98.949) (end 158 99) (width 0.2) (layer "F.Cu") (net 4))
 (segment (start 161.9375 99.5) (end 161.8875 99.55) (width 0.2) (layer "F.Cu") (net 4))
 (via (at 154 102) (size 0.6) (drill 0.3) (layers "F.Cu" "B.Cu") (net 4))
 (via (at 158 99) (size 0.6) (drill 0.3) (layers "F.Cu" "B.Cu") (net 4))
 (segment (start 156.896299 100.443115) (end 156.556886 100.103702) (width 0.2) (layer "B.Cu") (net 4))
 (segment (start 157.039259 100.586075) (end 156.896299 100.443115) (width 0.2) (layer "B.Cu") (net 4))
 (segment (start 156.13262 100.867376) (end 156.047768 100.952231) (width 0.2) (layer "B.Cu") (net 4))
 (segment (start 156.074523 99.96075) (end 155.989669 100.045603) (width 0.2) (layer "B.Cu") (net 4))
 (segment (start 156.047768 100.952231) (end 155 102) (width 0.2) (layer "B.Cu") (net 4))
 (segment (start 155 102) (end 154.916024 102) (width 0.2) (layer "B.Cu") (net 4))
 (segment (start 154.916024 102) (end 154 102) (width 0.2) (layer "B.Cu") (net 4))
 (segment (start 155.989669 100.385014) (end 156.13262 100.527965) (width 0.2) (layer "B.Cu") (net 4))
 (segment (start 158 99) (end 157.320562 99.679438) (width 0.2) (layer "B.Cu") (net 4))
 (segment (start 157.320562 100.01885) (end 157.463523 100.161811) (width 0.2) (layer "B.Cu") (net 4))
 (segment (start 156.556886 100.103702) (end 156.413934 99.96075) (width 0.2) (layer "B.Cu") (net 4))
 (segment (start 157.463522 100.501223) (end 157.378671 100.586075) (width 0.2) (layer "B.Cu") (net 4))
 (arc (start 156.413934 99.96075) (mid 156.244229 99.890455) (end 156.074523 99.96075) (width 0.2) (layer "B.Cu") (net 4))
 (arc (start 155.989669 100.045603) (mid 155.919375 100.215308) (end 155.989669 100.385014) (width 0.2) (layer "B.Cu") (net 4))
 (arc (start 156.13262 100.527965) (mid 156.202914 100.697671) (end 156.13262 100.867376) (width 0.2) (layer "B.Cu") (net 4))
 (arc (start 157.320562 99.679438) (mid 157.250266 99.849145) (end 157.320562 100.01885) (width 0.2) (layer "B.Cu") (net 4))
 (arc (start 157.463523 100.161811) (mid 157.533818 100.331516) (end 157.463522 100.501223) (width 0.2) (layer "B.Cu") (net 4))
 (arc (start 157.378671 100.586075) (mid 157.208964 100.656371) (end 157.039259 100.586075) (width 0.2) (layer "B.Cu") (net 4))
 (segment (start 160.576 101.076) (end 160 100.5) (width 0.2) (layer "F.Cu") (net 6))
 (segment (start 160 100.5) (end 159.6125 100.5) (width 0.2) (layer "F.Cu") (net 6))
 (segment (start 165.76 104) (end 164.659 105.101) (width 0.2) (layer "F.Cu") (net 6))
 (segment (start 161.751057 105.101) (end 160.576 103.925943) (width 0.2) (layer "F.Cu") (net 6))
 (segment (start 164.659 105.101) (end 161.751057 105.101) (width 0.2) (layer "F.Cu") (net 6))
 (segment (start 154 100.5) (end 159.6125 100.5) (width 0.2) (layer "F.Cu") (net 6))
 (segment (start 160.576 103.925943) (end 160.576 101.076) (width 0.2) (layer "F.Cu") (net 6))
 (segment (start 154.101 106.751057) (end 153.349943 106) (width 0.2) (layer "F.Cu") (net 12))
 (segment (start 156.998943 106.751057) (end 154.101 106.751057) (width 0.2) (layer "F.Cu") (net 12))
 (segment (start 153.349943 106) (end 152.5 106) (width 0.2) (layer "F.Cu") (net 12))
 (segment (start 157.75 106) (end 156.998943 106.751057) (width 0.2) (layer "F.Cu") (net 12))
 (segment (start 153.359943 107.99) (end 152.5 107.99) (width 0.2) (layer "F.Cu") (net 2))
 (segment (start 157.129 107.369) (end 153.980943 107.369) (width 0.2) (layer "F.Cu") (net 2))
 (segment (start 157.75 107.99) (end 157.129 107.369) (width 0.2) (layer "F.Cu") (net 2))
 (segment (start 153.980943 107.369) (end 153.359943 107.99) (width 0.2) (layer "F.Cu") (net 2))
 (segment (start 156.73 106) (end 156.73 105.680001) (width 0.2) (layer "F.Cu") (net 9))
 (segment (start 156.73 105.680001) (end 154.333549 103.28355) (width 0.2) (layer "F.Cu") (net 9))
 (segment (start 154.333549 103.28355) (end 154.28355 103.28355) (width 0.2) (layer "F.Cu") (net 9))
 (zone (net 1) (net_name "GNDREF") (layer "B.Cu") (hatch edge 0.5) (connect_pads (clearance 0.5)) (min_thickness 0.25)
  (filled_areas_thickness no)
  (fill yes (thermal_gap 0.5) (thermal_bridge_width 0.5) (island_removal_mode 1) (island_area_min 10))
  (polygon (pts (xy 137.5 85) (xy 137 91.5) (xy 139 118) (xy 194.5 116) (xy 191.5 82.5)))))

